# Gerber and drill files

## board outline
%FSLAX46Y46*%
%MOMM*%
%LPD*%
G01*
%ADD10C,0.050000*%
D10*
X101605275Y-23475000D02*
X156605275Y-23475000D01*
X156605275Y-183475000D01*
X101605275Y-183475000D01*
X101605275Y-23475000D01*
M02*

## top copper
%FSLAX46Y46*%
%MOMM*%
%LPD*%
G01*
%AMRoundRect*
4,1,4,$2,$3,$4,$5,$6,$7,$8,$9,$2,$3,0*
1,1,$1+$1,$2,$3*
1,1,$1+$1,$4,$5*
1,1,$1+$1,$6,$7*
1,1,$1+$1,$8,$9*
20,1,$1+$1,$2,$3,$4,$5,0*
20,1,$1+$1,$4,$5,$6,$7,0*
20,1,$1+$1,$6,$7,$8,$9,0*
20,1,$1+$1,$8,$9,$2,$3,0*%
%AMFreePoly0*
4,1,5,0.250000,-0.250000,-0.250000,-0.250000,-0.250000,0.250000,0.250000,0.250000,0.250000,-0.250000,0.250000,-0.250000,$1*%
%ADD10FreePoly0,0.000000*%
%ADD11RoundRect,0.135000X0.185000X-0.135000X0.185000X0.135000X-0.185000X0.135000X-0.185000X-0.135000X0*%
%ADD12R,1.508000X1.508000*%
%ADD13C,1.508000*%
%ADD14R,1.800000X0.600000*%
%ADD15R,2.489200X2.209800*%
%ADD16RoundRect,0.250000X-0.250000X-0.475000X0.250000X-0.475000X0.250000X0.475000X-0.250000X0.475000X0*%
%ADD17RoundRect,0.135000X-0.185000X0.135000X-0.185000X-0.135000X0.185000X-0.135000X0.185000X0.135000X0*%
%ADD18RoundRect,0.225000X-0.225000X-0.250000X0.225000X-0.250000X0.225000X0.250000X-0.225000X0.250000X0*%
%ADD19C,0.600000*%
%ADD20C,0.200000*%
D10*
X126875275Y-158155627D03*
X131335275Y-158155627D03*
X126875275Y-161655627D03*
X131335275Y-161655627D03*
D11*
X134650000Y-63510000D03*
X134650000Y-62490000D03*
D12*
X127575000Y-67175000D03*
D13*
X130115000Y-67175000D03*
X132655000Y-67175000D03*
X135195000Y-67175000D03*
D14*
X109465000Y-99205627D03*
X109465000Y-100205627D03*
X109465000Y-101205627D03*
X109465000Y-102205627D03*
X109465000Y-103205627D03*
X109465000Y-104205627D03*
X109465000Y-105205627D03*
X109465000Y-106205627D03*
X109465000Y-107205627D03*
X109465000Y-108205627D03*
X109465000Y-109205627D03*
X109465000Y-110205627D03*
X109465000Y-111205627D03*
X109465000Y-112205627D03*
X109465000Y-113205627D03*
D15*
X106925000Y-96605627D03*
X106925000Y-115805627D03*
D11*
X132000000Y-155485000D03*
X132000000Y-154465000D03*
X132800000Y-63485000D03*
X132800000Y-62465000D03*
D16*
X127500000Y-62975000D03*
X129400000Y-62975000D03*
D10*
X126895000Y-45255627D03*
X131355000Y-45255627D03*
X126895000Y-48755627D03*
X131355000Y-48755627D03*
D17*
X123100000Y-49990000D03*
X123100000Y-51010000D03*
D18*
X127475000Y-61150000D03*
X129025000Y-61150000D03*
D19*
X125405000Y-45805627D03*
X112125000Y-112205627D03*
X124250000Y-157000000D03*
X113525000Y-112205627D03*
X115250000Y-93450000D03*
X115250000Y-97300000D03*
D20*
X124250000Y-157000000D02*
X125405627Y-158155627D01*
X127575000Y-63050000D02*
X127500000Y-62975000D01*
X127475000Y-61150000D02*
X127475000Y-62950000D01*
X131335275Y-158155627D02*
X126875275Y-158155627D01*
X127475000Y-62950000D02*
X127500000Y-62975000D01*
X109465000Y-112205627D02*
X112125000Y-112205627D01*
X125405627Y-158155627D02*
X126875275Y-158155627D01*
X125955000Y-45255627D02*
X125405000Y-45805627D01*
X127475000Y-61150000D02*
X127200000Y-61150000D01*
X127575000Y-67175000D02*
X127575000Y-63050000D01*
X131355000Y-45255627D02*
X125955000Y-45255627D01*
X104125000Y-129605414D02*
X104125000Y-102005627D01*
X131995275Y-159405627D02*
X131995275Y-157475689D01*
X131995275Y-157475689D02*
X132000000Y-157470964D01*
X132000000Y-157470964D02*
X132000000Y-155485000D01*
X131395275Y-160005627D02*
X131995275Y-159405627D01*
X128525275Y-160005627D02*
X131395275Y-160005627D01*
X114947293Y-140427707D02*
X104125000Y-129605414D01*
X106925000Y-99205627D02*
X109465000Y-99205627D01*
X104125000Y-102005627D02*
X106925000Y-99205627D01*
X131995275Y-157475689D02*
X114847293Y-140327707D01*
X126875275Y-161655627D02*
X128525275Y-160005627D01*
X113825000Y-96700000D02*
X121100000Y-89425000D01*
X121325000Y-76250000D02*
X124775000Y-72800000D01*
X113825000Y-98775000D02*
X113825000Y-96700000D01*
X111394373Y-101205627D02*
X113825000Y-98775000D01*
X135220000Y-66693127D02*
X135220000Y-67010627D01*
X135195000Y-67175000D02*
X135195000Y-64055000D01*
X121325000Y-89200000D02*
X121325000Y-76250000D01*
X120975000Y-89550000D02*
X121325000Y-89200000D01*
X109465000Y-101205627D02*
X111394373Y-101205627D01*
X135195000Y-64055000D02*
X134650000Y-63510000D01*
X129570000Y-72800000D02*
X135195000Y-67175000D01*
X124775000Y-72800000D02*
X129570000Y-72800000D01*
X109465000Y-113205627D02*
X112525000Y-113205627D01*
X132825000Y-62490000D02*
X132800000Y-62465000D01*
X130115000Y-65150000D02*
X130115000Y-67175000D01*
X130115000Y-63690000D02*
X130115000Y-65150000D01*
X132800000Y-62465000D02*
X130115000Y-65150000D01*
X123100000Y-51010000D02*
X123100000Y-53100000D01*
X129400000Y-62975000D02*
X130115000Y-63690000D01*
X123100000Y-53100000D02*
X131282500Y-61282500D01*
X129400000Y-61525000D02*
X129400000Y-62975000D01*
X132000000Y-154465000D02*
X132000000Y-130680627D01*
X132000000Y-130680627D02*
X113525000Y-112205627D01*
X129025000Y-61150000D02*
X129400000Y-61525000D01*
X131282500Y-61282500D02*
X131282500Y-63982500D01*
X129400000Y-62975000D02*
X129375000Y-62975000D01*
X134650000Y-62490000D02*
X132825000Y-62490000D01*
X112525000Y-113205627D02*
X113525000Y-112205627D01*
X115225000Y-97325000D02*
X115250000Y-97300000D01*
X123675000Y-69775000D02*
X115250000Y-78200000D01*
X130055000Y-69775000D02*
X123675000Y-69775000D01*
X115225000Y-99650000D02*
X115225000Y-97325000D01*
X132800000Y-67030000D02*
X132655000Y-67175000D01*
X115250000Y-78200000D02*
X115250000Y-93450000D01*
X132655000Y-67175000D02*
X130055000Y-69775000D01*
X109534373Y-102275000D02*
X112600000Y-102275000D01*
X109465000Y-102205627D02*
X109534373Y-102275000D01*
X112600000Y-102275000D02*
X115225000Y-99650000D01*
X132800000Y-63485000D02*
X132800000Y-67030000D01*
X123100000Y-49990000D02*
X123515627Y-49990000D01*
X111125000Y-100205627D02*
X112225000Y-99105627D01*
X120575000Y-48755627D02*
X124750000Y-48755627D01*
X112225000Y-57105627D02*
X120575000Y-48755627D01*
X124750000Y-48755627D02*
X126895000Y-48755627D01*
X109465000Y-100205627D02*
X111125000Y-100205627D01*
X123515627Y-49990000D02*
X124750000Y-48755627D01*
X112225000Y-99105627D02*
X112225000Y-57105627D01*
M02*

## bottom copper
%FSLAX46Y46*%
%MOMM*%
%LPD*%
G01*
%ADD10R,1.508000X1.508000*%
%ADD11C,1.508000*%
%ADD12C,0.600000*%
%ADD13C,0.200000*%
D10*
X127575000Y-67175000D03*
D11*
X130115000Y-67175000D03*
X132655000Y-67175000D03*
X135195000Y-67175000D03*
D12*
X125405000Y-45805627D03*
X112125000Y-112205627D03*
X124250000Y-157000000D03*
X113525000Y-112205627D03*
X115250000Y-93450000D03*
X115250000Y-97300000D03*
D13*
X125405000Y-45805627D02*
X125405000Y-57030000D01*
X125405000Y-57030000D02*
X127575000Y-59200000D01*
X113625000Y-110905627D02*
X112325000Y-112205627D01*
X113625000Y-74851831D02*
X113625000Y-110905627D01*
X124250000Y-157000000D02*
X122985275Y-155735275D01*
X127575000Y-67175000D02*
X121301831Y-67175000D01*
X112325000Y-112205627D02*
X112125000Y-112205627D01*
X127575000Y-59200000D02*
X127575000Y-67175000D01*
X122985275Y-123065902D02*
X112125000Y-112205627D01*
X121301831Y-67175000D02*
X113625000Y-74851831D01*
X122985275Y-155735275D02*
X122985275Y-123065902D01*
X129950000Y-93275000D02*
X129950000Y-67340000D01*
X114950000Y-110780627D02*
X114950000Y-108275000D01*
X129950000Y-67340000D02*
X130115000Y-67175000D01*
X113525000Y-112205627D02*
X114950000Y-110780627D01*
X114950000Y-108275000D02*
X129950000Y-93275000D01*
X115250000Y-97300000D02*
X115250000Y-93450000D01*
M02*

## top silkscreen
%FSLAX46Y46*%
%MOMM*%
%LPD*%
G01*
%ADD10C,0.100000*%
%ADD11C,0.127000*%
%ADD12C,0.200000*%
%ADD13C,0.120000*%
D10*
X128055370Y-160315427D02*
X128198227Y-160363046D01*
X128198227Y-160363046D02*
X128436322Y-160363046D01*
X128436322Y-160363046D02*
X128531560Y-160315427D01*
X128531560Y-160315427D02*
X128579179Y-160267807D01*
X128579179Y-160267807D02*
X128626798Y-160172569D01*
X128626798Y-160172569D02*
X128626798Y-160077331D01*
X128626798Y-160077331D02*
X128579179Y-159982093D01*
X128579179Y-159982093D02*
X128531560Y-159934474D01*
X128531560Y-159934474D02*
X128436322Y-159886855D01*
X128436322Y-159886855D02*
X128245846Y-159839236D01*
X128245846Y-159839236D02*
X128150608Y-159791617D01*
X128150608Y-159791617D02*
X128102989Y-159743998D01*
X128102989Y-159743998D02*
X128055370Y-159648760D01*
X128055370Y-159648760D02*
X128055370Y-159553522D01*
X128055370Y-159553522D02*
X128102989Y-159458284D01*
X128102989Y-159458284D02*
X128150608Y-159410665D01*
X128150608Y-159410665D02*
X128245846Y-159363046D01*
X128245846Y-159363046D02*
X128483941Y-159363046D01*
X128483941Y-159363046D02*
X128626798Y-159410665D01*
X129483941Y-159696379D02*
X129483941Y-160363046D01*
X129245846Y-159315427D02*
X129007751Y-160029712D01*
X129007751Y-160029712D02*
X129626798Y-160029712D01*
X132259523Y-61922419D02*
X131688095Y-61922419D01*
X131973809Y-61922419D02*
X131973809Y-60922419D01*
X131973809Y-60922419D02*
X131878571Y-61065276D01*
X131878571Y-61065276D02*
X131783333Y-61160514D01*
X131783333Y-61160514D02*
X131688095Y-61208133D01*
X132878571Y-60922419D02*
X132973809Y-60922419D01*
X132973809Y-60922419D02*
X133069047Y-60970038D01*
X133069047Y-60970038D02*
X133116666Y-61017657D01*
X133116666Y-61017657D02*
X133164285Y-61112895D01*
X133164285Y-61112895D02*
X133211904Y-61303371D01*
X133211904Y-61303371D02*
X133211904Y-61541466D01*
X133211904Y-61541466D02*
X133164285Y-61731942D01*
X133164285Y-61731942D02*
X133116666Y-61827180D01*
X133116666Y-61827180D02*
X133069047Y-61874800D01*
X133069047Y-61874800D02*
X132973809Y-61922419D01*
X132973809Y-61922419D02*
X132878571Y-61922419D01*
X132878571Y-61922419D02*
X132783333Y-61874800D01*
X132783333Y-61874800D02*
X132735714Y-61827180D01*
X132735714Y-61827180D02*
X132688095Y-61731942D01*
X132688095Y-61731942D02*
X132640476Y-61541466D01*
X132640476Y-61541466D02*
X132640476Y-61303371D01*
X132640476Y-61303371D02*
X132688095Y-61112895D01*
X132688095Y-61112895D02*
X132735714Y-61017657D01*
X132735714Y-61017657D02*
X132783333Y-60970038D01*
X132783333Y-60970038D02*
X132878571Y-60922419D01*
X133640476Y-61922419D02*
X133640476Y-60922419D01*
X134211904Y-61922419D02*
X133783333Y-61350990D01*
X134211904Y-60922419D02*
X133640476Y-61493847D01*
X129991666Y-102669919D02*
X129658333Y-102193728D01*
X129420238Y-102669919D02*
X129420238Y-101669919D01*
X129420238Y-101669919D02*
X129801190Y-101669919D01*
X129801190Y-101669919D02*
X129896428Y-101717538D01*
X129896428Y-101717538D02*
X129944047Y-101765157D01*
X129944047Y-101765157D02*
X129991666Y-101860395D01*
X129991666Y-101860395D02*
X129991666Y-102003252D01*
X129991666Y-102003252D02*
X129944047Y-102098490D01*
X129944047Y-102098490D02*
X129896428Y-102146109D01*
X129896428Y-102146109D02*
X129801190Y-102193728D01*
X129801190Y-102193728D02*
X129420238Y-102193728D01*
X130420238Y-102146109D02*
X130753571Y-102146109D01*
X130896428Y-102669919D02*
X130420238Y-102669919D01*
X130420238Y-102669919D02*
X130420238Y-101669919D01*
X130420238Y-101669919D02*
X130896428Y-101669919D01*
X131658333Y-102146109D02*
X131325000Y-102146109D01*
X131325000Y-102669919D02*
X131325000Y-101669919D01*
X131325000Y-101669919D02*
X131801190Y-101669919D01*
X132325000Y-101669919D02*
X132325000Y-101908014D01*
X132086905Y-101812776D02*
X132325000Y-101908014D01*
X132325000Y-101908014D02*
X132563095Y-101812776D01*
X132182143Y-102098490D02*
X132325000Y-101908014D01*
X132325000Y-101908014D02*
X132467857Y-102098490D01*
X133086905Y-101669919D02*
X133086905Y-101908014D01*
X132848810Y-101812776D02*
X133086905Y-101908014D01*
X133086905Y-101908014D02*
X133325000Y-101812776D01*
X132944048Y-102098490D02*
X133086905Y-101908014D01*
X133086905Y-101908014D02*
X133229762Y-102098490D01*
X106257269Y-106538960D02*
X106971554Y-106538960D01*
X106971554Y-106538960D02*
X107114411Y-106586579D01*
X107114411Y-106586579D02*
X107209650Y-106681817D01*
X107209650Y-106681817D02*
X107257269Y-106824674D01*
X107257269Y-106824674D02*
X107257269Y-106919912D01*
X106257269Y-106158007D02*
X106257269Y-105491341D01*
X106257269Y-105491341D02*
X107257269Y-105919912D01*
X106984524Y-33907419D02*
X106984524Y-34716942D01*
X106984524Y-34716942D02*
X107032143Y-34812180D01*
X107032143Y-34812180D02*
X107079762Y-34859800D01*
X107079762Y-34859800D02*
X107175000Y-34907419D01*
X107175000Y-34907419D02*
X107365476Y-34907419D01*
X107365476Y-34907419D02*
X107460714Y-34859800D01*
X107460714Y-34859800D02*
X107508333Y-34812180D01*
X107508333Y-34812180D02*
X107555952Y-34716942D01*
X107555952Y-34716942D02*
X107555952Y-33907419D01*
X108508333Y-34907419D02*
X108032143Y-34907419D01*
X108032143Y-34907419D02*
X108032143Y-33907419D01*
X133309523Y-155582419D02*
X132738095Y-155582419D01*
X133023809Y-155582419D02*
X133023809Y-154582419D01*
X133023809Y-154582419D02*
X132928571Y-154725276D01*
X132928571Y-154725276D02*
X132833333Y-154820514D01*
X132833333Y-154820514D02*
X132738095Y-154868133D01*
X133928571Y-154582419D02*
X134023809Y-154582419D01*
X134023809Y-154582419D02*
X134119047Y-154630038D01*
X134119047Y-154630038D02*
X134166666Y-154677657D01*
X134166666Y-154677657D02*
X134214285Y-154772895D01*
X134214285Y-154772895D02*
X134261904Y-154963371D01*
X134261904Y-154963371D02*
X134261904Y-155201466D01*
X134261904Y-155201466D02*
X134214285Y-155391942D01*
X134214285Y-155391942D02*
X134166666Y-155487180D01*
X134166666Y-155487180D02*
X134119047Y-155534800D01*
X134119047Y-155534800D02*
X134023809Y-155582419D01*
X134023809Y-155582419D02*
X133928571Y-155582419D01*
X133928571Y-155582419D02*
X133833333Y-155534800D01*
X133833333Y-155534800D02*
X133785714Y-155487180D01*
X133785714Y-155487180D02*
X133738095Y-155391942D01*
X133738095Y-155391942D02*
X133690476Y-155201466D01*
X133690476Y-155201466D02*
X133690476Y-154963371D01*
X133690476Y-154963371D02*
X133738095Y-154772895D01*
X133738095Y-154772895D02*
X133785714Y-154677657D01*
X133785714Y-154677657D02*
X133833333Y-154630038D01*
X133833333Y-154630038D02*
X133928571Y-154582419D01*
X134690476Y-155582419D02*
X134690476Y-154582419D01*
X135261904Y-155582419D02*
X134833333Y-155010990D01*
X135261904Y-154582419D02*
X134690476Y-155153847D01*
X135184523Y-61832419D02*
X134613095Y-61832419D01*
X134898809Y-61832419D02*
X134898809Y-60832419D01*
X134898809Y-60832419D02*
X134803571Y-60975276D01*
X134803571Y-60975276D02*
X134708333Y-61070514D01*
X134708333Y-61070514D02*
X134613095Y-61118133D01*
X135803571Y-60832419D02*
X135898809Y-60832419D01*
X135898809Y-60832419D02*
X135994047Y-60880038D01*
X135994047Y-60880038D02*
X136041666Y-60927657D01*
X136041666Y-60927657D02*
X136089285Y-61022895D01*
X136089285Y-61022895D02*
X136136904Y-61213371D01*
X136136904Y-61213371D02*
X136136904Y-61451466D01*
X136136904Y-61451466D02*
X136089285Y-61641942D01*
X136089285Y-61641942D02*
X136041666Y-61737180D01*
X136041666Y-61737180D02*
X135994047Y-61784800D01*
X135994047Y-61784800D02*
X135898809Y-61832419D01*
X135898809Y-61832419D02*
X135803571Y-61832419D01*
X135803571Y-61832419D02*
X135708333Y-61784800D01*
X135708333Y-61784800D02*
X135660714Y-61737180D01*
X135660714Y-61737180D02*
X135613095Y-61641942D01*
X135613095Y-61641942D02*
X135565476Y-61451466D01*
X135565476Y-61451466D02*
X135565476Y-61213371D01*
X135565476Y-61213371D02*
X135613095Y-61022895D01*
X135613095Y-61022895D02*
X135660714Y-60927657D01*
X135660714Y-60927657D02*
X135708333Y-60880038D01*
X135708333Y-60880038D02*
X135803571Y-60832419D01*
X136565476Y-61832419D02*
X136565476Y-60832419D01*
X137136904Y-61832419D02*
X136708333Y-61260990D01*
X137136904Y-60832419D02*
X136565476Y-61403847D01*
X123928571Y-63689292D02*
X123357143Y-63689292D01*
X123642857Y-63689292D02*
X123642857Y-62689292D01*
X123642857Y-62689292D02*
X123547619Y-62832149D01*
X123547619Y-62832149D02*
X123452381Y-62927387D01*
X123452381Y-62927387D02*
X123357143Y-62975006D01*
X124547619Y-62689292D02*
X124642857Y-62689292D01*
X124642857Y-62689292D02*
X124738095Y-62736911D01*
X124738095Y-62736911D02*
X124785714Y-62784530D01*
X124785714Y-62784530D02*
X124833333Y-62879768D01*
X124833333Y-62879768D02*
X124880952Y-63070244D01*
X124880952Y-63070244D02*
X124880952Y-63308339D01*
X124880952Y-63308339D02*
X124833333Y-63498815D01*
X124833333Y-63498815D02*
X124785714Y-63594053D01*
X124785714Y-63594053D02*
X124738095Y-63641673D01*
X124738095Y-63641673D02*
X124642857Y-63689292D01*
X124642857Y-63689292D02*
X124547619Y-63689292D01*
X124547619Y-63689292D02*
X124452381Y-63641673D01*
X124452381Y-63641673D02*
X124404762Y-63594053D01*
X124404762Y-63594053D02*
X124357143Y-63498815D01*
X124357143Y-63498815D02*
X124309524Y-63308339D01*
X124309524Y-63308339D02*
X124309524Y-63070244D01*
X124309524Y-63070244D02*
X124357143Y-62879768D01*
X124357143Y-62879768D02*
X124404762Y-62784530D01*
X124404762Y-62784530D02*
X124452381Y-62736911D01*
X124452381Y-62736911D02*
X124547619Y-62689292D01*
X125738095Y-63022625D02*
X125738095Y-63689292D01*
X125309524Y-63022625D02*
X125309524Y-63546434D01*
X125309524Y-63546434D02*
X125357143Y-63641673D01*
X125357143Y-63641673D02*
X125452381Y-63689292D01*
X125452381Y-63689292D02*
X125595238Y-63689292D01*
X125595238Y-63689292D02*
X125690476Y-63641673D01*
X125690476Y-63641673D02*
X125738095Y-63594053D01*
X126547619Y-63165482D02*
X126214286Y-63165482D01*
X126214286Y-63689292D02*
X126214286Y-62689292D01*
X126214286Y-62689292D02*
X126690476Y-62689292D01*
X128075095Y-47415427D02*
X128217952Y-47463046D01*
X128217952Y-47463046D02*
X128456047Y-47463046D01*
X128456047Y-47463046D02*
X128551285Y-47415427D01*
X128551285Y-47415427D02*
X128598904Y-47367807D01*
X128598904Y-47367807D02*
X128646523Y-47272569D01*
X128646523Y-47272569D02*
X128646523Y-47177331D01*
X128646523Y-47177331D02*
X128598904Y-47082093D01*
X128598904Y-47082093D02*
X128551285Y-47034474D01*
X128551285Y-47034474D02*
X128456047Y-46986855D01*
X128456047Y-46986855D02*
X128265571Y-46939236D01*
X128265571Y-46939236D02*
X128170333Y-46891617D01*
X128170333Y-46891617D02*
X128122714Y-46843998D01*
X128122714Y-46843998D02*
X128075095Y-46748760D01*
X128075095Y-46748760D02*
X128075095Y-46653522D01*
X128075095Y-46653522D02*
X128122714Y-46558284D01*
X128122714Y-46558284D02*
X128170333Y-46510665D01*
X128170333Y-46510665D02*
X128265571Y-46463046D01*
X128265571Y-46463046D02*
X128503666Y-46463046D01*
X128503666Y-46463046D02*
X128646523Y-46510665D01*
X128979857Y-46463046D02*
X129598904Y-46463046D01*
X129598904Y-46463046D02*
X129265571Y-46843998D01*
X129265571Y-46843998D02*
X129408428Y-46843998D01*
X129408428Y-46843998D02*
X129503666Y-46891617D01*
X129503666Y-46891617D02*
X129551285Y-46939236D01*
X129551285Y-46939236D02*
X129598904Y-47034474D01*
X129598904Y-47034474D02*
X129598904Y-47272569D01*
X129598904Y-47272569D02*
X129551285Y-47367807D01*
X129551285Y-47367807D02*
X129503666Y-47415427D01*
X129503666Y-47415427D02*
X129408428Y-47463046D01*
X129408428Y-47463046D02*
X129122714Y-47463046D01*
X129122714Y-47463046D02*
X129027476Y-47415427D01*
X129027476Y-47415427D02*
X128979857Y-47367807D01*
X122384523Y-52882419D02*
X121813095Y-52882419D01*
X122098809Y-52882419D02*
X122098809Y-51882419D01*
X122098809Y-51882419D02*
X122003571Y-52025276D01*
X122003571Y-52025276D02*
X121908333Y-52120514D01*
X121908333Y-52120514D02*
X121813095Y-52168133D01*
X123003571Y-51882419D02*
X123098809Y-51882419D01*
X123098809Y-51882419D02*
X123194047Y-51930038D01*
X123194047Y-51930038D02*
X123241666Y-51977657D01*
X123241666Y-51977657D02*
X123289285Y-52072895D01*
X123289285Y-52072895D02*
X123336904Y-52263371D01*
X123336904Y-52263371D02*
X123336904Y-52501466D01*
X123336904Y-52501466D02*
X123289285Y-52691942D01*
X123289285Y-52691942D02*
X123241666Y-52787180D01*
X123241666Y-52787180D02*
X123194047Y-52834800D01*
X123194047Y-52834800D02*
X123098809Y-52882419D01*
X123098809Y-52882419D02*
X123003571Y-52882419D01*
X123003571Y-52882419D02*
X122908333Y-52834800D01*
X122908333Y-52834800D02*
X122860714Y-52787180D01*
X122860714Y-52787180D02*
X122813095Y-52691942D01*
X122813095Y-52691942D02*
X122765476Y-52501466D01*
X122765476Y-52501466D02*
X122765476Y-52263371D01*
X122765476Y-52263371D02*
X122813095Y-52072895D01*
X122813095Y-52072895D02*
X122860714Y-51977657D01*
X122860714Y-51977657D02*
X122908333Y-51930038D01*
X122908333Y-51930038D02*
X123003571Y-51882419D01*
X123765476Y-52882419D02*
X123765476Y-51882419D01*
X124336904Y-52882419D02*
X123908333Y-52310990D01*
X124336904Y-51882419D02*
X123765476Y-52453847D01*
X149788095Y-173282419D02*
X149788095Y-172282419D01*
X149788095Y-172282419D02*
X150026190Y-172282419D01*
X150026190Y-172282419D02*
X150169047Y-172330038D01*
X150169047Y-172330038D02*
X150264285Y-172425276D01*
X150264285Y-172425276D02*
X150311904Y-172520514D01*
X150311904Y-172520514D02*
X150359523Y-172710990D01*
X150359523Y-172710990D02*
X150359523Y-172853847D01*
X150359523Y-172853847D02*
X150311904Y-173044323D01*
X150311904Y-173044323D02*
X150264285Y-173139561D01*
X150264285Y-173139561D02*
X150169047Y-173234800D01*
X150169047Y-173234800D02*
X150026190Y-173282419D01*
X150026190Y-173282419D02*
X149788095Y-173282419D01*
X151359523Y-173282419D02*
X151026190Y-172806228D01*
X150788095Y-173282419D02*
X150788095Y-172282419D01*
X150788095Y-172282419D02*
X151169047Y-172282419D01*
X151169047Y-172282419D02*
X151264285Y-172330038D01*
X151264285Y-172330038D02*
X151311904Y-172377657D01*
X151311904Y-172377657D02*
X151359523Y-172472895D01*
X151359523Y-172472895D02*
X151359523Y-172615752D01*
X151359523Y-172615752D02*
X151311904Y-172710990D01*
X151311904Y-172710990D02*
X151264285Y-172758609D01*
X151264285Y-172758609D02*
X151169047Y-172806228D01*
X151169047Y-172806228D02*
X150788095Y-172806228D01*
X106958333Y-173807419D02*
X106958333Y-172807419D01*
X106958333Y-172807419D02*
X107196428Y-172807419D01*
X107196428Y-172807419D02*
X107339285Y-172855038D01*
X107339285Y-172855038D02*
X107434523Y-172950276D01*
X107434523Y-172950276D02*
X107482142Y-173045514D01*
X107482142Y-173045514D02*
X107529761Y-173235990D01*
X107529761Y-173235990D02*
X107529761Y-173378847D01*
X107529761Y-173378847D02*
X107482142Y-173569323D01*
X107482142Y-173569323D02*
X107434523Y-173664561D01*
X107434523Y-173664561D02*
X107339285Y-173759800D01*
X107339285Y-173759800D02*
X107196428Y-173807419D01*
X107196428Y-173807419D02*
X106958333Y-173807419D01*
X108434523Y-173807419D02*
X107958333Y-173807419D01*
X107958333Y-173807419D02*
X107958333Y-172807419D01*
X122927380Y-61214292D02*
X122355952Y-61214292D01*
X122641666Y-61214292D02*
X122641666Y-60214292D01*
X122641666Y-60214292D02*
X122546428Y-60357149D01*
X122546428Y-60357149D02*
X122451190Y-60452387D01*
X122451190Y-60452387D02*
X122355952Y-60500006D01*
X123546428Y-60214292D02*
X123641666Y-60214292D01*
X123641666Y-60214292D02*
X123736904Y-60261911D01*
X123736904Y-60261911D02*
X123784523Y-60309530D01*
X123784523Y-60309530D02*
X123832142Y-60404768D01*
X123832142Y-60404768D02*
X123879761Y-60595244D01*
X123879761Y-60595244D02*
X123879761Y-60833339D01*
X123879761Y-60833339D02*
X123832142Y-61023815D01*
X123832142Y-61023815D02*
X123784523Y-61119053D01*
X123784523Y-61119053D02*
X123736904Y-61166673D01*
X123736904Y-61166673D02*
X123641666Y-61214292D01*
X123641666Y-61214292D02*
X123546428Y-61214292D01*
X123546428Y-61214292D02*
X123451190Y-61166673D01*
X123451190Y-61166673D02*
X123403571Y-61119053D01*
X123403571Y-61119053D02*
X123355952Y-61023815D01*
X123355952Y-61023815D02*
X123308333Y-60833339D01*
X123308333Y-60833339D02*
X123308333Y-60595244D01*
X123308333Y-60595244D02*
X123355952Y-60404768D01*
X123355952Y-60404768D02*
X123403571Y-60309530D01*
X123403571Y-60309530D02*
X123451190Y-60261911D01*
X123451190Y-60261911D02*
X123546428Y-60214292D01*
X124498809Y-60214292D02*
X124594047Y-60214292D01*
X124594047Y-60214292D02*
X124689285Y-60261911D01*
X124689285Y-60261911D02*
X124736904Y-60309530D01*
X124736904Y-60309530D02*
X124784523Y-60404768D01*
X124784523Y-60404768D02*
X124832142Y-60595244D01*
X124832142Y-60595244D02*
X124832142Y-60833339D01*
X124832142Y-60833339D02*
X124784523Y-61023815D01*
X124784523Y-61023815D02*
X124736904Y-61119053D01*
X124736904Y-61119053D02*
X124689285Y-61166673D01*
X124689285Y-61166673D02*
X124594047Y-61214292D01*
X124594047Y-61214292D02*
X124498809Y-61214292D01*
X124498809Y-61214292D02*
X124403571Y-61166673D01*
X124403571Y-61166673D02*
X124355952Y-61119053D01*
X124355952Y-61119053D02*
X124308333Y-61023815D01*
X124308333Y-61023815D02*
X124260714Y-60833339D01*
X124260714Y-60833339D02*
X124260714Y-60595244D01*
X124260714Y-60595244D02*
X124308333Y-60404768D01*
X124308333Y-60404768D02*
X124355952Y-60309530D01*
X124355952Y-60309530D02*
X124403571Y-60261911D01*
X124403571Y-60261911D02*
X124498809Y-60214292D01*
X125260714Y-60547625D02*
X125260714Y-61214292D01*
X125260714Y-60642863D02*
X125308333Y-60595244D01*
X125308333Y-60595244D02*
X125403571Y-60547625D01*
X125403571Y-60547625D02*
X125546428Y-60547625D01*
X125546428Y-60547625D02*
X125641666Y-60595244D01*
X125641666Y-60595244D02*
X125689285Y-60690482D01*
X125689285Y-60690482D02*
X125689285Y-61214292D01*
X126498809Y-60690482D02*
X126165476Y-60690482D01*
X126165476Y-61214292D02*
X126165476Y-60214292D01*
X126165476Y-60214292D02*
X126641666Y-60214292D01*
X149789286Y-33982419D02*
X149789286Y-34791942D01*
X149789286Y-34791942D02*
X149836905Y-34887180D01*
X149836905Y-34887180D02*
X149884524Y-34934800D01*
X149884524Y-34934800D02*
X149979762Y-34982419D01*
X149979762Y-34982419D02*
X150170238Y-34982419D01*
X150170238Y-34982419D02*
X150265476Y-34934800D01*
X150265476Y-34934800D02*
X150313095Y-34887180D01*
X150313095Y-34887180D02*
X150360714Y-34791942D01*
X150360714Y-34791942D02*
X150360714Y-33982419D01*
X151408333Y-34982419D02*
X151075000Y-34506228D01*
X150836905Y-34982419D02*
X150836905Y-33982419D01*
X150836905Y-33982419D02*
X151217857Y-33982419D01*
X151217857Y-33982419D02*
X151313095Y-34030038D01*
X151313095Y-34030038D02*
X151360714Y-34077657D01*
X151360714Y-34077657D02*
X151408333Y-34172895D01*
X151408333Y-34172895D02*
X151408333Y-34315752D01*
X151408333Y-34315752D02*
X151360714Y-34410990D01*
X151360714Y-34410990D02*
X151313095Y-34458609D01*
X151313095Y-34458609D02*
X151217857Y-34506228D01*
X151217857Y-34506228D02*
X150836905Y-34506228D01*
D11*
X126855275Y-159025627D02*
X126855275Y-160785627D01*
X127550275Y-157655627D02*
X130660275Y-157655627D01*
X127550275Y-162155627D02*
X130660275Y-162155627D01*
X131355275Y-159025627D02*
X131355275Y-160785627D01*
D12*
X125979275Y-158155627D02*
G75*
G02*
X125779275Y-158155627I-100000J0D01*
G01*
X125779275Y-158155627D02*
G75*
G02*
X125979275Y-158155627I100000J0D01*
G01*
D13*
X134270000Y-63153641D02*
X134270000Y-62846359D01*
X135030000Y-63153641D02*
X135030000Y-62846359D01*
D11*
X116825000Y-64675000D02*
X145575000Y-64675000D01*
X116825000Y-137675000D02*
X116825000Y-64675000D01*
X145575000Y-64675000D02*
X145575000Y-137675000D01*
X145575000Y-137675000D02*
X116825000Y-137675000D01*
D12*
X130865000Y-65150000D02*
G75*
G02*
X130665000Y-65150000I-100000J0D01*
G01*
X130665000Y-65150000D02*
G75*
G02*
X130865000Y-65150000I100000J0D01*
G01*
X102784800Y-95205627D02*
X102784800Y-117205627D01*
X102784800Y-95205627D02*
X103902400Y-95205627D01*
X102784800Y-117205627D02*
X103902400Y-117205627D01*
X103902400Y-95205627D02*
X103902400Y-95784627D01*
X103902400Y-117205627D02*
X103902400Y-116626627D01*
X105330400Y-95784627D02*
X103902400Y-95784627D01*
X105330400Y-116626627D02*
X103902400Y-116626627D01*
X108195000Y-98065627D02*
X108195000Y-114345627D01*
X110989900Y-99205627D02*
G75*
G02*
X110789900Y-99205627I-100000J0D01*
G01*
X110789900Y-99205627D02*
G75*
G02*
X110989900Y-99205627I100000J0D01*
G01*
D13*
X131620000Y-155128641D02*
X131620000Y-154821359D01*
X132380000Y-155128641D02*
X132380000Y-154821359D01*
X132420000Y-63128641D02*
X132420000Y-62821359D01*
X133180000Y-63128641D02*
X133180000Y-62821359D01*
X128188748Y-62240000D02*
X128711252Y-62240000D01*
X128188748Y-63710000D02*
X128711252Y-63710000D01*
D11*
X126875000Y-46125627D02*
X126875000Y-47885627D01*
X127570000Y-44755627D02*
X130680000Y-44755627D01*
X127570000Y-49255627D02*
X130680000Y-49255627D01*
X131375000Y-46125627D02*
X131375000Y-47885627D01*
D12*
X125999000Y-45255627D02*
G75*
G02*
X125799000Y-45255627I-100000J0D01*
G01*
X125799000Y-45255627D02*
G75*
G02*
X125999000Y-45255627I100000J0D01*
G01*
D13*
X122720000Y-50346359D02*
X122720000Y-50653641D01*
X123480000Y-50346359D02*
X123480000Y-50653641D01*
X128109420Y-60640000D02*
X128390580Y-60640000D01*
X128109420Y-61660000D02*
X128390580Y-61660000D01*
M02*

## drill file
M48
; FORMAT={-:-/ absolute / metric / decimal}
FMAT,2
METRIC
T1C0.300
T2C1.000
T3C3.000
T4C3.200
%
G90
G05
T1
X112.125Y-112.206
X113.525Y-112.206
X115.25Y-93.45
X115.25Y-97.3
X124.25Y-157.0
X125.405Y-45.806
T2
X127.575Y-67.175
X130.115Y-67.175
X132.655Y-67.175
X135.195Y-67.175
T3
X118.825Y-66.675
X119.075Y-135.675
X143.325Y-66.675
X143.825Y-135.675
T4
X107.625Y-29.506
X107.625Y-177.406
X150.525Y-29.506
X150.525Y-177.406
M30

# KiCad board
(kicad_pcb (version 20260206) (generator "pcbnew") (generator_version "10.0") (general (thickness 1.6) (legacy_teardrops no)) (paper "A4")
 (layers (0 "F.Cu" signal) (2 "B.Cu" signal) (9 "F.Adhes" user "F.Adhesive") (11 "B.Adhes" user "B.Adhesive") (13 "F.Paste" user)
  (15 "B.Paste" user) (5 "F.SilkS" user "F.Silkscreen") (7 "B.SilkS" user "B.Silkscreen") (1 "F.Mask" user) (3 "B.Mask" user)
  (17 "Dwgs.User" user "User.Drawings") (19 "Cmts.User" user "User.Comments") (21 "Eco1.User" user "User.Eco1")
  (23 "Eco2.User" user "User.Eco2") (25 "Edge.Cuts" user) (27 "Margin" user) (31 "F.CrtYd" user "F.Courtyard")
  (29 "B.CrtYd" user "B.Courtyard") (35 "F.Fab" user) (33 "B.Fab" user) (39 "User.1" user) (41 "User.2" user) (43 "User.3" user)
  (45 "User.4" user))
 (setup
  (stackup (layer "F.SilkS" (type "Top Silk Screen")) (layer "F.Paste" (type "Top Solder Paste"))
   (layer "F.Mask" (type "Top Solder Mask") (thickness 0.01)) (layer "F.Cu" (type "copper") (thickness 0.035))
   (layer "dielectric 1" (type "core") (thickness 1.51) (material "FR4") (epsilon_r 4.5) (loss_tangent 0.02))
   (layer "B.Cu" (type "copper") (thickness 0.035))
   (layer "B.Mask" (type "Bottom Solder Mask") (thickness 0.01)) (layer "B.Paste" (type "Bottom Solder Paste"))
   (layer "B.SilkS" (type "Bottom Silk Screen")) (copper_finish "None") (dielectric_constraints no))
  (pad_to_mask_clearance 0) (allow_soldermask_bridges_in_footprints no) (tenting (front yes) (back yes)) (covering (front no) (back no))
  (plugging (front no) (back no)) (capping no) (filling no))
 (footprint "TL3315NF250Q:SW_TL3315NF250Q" (layer "F.Cu") (at 129.105275 159.905627)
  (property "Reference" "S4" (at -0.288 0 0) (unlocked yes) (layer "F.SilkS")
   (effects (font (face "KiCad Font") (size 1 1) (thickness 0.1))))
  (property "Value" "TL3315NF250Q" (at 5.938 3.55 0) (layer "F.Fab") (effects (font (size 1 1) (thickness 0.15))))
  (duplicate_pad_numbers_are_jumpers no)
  (fp_line (start -2.25 -0.88) (end -2.25 0.88) (stroke (width 0.127) (type solid)) (layer "F.SilkS"))
  (fp_line (start -1.555 -2.25) (end 1.555 -2.25) (stroke (width 0.127) (type solid)) (layer "F.SilkS"))
  (fp_line (start -1.555 2.25) (end 1.555 2.25) (stroke (width 0.127) (type solid)) (layer "F.SilkS"))
  (fp_line (start 2.25 -0.88) (end 2.25 0.88) (stroke (width 0.127) (type solid)) (layer "F.SilkS"))
  (fp_circle (center -3.226 -1.75) (end -3.126 -1.75) (stroke (width 0.2) (type solid)) (fill no) (layer "F.SilkS"))
  (pad "1" smd custom (at -2.23 -1.75) (size 0.5 0.5) (layers "F.Cu") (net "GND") (options (clearance outline) (anchor rect)) (primitives))
  (pad "2" smd custom (at 2.23 -1.75) (size 0.5 0.5) (layers "F.Cu") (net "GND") (options (clearance outline) (anchor rect)) (primitives))
  (pad "3" smd custom (at -2.23 1.75) (size 0.5 0.5) (layers "F.Cu") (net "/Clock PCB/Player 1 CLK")
   (options (clearance outline) (anchor rect)) (primitives))
  (pad "4" smd custom (at 2.23 1.75) (size 0.5 0.5) (layers "F.Cu") (options (clearance outline) (anchor rect)) (primitives)))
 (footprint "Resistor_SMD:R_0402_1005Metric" (layer "F.Cu") (at 134.65 63 90)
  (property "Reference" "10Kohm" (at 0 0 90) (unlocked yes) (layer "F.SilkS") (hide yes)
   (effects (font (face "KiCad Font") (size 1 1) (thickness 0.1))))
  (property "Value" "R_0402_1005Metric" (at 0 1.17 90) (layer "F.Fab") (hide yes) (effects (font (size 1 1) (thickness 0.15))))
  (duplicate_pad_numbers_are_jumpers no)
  (fp_line (start -0.153641 -0.38) (end 0.153641 -0.38) (stroke (width 0.12) (type solid)) (layer "F.SilkS"))
  (fp_line (start -0.153641 0.38) (end 0.153641 0.38) (stroke (width 0.12) (type solid)) (layer "F.SilkS"))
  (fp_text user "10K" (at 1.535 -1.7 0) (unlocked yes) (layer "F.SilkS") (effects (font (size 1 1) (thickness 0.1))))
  (pad "1" smd roundrect (at -0.51 0 90) (size 0.54 0.64) (layers "F.Cu" "F.Mask" "F.Paste") (roundrect_rratio 0.25) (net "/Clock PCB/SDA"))
  (pad "2" smd roundrect (at 0.51 0 90) (size 0.54 0.64) (layers "F.Cu" "F.Mask" "F.Paste") (roundrect_rratio 0.25) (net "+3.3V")))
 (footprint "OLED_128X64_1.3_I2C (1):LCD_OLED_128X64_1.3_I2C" (layer "F.Cu") (at 131.325 101.675)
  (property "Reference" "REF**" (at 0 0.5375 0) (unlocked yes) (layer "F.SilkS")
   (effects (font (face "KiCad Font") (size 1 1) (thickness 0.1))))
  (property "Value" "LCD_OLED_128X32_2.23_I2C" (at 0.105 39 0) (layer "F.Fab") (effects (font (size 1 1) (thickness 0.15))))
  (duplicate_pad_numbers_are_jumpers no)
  (fp_line (start -14.5 -37) (end 14.25 -37) (stroke (width 0.127) (type solid)) (layer "F.SilkS"))
  (fp_line (start -14.5 36) (end -14.5 -37) (stroke (width 0.127) (type solid)) (layer "F.SilkS"))
  (fp_line (start 14.25 -37) (end 14.25 36) (stroke (width 0.127) (type solid)) (layer "F.SilkS"))
  (fp_line (start 14.25 36) (end -14.5 36) (stroke (width 0.127) (type solid)) (layer "F.SilkS"))
  (fp_circle (center -0.56 -36.525) (end -0.46 -36.525) (stroke (width 0.2) (type solid)) (fill no) (layer "F.SilkS"))
  (pad "" np_thru_hole circle (at -12.5 -35) (size 3 3) (drill 3) (layers "*.Cu" "*.Mask"))
  (pad "" np_thru_hole circle (at -12.25 34) (size 3 3) (drill 3) (layers "*.Cu" "*.Mask"))
  (pad "" np_thru_hole circle (at 12 -35) (size 3 3) (drill 3) (layers "*.Cu" "*.Mask"))
  (pad "" np_thru_hole circle (at 12.5 34) (size 3 3) (drill 3) (layers "*.Cu" "*.Mask"))
  (pad "1" thru_hole rect (at -3.75 -34.5) (size 1.508 1.508) (drill 1) (layers "*.Cu" "*.Mask") (remove_unused_layers no) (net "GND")
   (solder_mask_margin 0.102))
  (pad "2" thru_hole circle (at -1.21 -34.5) (size 1.508 1.508) (drill 1) (layers "*.Cu" "*.Mask") (remove_unused_layers no) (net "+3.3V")
   (solder_mask_margin 0.102))
  (pad "3" thru_hole circle (at 1.33 -34.5) (size 1.508 1.508) (drill 1) (layers "*.Cu" "*.Mask") (remove_unused_layers no) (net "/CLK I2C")
   (solder_mask_margin 0.102))
  (pad "4" thru_hole circle (at 3.87 -34.5) (size 1.508 1.508) (drill 1) (layers "*.Cu" "*.Mask") (remove_unused_layers no)
   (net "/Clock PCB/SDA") (solder_mask_margin 0.102)))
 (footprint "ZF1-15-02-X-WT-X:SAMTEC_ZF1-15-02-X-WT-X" (layer "F.Cu") (at 105.4899 106.205627 -90)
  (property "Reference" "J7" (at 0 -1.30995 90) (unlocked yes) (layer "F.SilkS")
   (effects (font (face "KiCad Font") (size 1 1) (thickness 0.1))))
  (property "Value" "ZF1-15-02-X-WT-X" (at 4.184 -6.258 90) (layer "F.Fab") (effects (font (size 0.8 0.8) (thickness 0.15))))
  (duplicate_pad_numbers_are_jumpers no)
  (fp_line (start -11 2.7051) (end 11 2.7051) (stroke (width 0.2) (type solid)) (layer "F.SilkS"))
  (fp_line (start -11 2.7051) (end -11 1.5875) (stroke (width 0.2) (type solid)) (layer "F.SilkS"))
  (fp_line (start 11 2.7051) (end 11 1.5875) (stroke (width 0.2) (type solid)) (layer "F.SilkS"))
  (fp_line (start -11 1.5875) (end -10.421 1.5875) (stroke (width 0.2) (type solid)) (layer "F.SilkS"))
  (fp_line (start 11 1.5875) (end 10.421 1.5875) (stroke (width 0.2) (type solid)) (layer "F.SilkS"))
  (fp_line (start -10.421 0.1595) (end -10.421 1.5875) (stroke (width 0.2) (type solid)) (layer "F.SilkS"))
  (fp_line (start 10.421 0.1595) (end 10.421 1.5875) (stroke (width 0.2) (type solid)) (layer "F.SilkS"))
  (fp_line (start -8.14 -2.7051) (end 8.14 -2.7051) (stroke (width 0.2) (type solid)) (layer "F.SilkS"))
  (fp_circle (center -7 -5.4) (end -6.9 -5.4) (stroke (width 0.2) (type solid)) (fill no) (layer "F.SilkS"))
  (pad "01" smd rect (at -7 -3.9751 270) (size 0.6 1.8) (layers "F.Cu" "F.Mask" "F.Paste") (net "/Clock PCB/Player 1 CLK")
   (solder_mask_margin 0.102))
  (pad "02" smd rect (at -6 -3.9751 270) (size 0.6 1.8) (layers "F.Cu" "F.Mask" "F.Paste") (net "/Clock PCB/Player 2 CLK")
   (solder_mask_margin 0.102))
  (pad "03" smd rect (at -5 -3.9751 270) (size 0.6 1.8) (layers "F.Cu" "F.Mask" "F.Paste") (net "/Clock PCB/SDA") (solder_mask_margin 0.102))
  (pad "04" smd rect (at -4 -3.9751 270) (size 0.6 1.8) (layers "F.Cu" "F.Mask" "F.Paste") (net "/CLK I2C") (solder_mask_margin 0.102))
  (pad "05" smd rect (at -3 -3.9751 270) (size 0.6 1.8) (layers "F.Cu" "F.Mask" "F.Paste") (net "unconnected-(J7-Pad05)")
   (solder_mask_margin 0.102))
  (pad "06" smd rect (at -2 -3.9751 270) (size 0.6 1.8) (layers "F.Cu" "F.Mask" "F.Paste") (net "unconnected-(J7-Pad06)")
   (solder_mask_margin 0.102))
  (pad "07" smd rect (at -1 -3.9751 270) (size 0.6 1.8) (layers "F.Cu" "F.Mask" "F.Paste") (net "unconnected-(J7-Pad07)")
   (solder_mask_margin 0.102))
  (pad "08" smd rect (at 0 -3.9751 270) (size 0.6 1.8) (layers "F.Cu" "F.Mask" "F.Paste") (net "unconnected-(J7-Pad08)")
   (solder_mask_margin 0.102))
  (pad "09" smd rect (at 1 -3.9751 270) (size 0.6 1.8) (layers "F.Cu" "F.Mask" "F.Paste") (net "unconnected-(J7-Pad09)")
   (solder_mask_margin 0.102))
  (pad "10" smd rect (at 2 -3.9751 270) (size 0.6 1.8) (layers "F.Cu" "F.Mask" "F.Paste") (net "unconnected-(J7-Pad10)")
   (solder_mask_margin 0.102))
  (pad "11" smd rect (at 3 -3.9751 270) (size 0.6 1.8) (layers "F.Cu" "F.Mask" "F.Paste") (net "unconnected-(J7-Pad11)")
   (solder_mask_margin 0.102))
  (pad "12" smd rect (at 4 -3.9751 270) (size 0.6 1.8) (layers "F.Cu" "F.Mask" "F.Paste") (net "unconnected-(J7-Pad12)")
   (solder_mask_margin 0.102))
  (pad "13" smd rect (at 5 -3.9751 270) (size 0.6 1.8) (layers "F.Cu" "F.Mask" "F.Paste") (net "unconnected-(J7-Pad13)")
   (solder_mask_margin 0.102))
  (pad "14" smd rect (at 6 -3.9751 270) (size 0.6 1.8) (layers "F.Cu" "F.Mask" "F.Paste") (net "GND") (solder_mask_margin 0.102))
  (pad "15" smd rect (at 7 -3.9751 270) (size 0.6 1.8) (layers "F.Cu" "F.Mask" "F.Paste") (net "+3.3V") (solder_mask_margin 0.102))
  (pad "MP1" smd rect (at -9.6 -1.4351 270) (size 2.2098 2.4892) (layers "F.Cu" "F.Mask" "F.Paste") (solder_mask_margin 0.102))
  (pad "MP2" smd rect (at 9.6 -1.4351 270) (size 2.2098 2.4892) (layers "F.Cu" "F.Mask" "F.Paste") (solder_mask_margin 0.102)))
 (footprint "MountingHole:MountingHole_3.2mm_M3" (layer "F.Cu") (at 107.625 29.505627)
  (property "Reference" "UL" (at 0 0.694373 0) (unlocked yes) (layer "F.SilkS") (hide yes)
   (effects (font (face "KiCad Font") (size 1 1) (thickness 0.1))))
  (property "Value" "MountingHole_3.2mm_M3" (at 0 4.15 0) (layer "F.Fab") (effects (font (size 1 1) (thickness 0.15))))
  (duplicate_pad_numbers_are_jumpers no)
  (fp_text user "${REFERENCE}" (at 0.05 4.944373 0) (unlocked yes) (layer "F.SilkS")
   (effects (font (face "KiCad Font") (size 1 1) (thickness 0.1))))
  (pad "" np_thru_hole circle (at 0 0) (size 3.2 3.2) (drill 3.2) (layers "*.Cu" "*.Mask")))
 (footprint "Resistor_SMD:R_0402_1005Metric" (layer "F.Cu") (at 132 154.975 90)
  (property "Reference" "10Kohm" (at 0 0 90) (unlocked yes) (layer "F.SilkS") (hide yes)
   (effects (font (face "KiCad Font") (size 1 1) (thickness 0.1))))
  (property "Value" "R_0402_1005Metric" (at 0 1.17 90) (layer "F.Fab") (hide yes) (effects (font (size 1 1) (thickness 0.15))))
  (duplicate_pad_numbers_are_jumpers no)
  (fp_line (start -0.153641 -0.38) (end 0.153641 -0.38) (stroke (width 0.12) (type solid)) (layer "F.SilkS"))
  (fp_line (start -0.153641 0.38) (end 0.153641 0.38) (stroke (width 0.12) (type solid)) (layer "F.SilkS"))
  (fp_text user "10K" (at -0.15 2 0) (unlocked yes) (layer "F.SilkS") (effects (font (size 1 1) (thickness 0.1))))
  (pad "1" smd roundrect (at -0.51 0 90) (size 0.54 0.64) (layers "F.Cu" "F.Mask" "F.Paste") (roundrect_rratio 0.25)
   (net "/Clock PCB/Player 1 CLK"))
  (pad "2" smd roundrect (at 0.51 0 90) (size 0.54 0.64) (layers "F.Cu" "F.Mask" "F.Paste") (roundrect_rratio 0.25) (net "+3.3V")))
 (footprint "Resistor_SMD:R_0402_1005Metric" (layer "F.Cu") (at 132.8 62.975 90)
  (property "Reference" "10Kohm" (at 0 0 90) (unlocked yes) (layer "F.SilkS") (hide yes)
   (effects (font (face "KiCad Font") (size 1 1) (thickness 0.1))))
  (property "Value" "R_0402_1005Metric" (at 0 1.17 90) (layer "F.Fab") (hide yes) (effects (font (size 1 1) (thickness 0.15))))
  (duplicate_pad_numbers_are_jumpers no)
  (fp_line (start -0.153641 -0.38) (end 0.153641 -0.38) (stroke (width 0.12) (type solid)) (layer "F.SilkS"))
  (fp_line (start -0.153641 0.38) (end 0.153641 0.38) (stroke (width 0.12) (type solid)) (layer "F.SilkS"))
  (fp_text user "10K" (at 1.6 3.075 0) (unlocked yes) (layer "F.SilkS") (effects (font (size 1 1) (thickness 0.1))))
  (pad "1" smd roundrect (at -0.51 0 90) (size 0.54 0.64) (layers "F.Cu" "F.Mask" "F.Paste") (roundrect_rratio 0.25) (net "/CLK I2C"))
  (pad "2" smd roundrect (at 0.51 0 90) (size 0.54 0.64) (layers "F.Cu" "F.Mask" "F.Paste") (roundrect_rratio 0.25) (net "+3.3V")))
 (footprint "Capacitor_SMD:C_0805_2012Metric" (layer "F.Cu") (at 128.45 62.975)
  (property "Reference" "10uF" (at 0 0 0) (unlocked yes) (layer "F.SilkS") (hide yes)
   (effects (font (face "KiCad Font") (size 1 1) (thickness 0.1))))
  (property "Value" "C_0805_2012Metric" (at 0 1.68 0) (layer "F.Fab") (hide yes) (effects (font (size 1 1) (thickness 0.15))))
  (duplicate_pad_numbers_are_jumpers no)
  (fp_line (start -0.261252 -0.735) (end 0.261252 -0.735) (stroke (width 0.12) (type solid)) (layer "F.SilkS"))
  (fp_line (start -0.261252 0.735) (end 0.261252 0.735) (stroke (width 0.12) (type solid)) (layer "F.SilkS"))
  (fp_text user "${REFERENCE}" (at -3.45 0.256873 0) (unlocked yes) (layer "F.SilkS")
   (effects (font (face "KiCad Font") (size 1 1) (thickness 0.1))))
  (pad "1" smd roundrect (at -0.95 0) (size 1 1.45) (layers "F.Cu" "F.Mask" "F.Paste") (roundrect_rratio 0.25) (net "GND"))
  (pad "2" smd roundrect (at 0.95 0) (size 1 1.45) (layers "F.Cu" "F.Mask" "F.Paste") (roundrect_rratio 0.25) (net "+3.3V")))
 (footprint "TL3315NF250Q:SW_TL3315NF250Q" (layer "F.Cu") (at 129.125 47.005627)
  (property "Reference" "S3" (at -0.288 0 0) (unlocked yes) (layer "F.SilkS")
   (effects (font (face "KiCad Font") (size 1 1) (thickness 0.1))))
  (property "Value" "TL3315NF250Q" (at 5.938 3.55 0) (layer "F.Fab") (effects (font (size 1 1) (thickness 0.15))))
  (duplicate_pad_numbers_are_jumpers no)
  (fp_line (start -2.25 -0.88) (end -2.25 0.88) (stroke (width 0.127) (type solid)) (layer "F.SilkS"))
  (fp_line (start -1.555 -2.25) (end 1.555 -2.25) (stroke (width 0.127) (type solid)) (layer "F.SilkS"))
  (fp_line (start -1.555 2.25) (end 1.555 2.25) (stroke (width 0.127) (type solid)) (layer "F.SilkS"))
  (fp_line (start 2.25 -0.88) (end 2.25 0.88) (stroke (width 0.127) (type solid)) (layer "F.SilkS"))
  (fp_circle (center -3.226 -1.75) (end -3.126 -1.75) (stroke (width 0.2) (type solid)) (fill no) (layer "F.SilkS"))
  (pad "1" smd custom (at -2.23 -1.75) (size 0.5 0.5) (layers "F.Cu") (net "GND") (options (clearance outline) (anchor rect)) (primitives))
  (pad "2" smd custom (at 2.23 -1.75) (size 0.5 0.5) (layers "F.Cu") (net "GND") (options (clearance outline) (anchor rect)) (primitives))
  (pad "3" smd custom (at -2.23 1.75) (size 0.5 0.5) (layers "F.Cu") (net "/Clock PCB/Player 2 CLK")
   (options (clearance outline) (anchor rect)) (primitives))
  (pad "4" smd custom (at 2.23 1.75) (size 0.5 0.5) (layers "F.Cu") (options (clearance outline) (anchor rect)) (primitives)))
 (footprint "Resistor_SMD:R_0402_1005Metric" (layer "F.Cu") (at 123.1 50.5 -90)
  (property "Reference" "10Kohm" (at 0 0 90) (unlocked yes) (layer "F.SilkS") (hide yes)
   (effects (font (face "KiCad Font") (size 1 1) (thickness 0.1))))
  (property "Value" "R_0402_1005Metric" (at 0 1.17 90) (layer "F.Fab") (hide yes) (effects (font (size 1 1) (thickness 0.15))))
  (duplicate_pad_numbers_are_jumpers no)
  (fp_line (start -0.153641 0.38) (end 0.153641 0.38) (stroke (width 0.12) (type solid)) (layer "F.SilkS"))
  (fp_line (start -0.153641 -0.38) (end 0.153641 -0.38) (stroke (width 0.12) (type solid)) (layer "F.SilkS"))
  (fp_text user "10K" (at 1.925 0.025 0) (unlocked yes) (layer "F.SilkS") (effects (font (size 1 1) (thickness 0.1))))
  (pad "1" smd roundrect (at -0.51 0 270) (size 0.54 0.64) (layers "F.Cu" "F.Mask" "F.Paste") (roundrect_rratio 0.25)
   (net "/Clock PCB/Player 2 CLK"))
  (pad "2" smd roundrect (at 0.51 0 270) (size 0.54 0.64) (layers "F.Cu" "F.Mask" "F.Paste") (roundrect_rratio 0.25) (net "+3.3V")))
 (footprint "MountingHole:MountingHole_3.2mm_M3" (layer "F.Cu") (at 150.525 177.405627)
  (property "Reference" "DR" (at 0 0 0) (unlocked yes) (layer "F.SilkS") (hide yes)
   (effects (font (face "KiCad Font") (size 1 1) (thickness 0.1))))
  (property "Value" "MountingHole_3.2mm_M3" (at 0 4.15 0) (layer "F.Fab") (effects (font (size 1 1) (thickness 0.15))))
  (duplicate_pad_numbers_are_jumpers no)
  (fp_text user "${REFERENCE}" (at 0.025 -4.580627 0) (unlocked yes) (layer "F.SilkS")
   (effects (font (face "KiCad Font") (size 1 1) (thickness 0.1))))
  (pad "" np_thru_hole circle (at 0 0) (size 3.2 3.2) (drill 3.2) (layers "*.Cu" "*.Mask")))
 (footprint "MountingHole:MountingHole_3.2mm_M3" (layer "F.Cu") (at 107.625 177.405627)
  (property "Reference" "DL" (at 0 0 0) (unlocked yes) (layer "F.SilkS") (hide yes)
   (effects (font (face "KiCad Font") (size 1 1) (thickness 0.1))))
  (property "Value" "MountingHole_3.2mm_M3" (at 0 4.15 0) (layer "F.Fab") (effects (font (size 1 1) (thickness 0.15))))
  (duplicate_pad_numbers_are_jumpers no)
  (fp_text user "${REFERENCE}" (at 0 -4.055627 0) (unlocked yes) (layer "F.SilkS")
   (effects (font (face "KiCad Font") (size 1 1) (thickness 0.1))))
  (pad "" np_thru_hole circle (at 0 0) (size 3.2 3.2) (drill 3.2) (layers "*.Cu" "*.Mask")))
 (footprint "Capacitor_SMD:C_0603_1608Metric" (layer "F.Cu") (at 128.25 61.15)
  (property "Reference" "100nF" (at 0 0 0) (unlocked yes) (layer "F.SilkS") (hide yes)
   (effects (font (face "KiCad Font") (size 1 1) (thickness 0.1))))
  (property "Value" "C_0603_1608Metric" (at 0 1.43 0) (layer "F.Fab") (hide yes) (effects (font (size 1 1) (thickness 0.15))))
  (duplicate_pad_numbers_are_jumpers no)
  (fp_line (start -0.14058 -0.51) (end 0.14058 -0.51) (stroke (width 0.12) (type solid)) (layer "F.SilkS"))
  (fp_line (start -0.14058 0.51) (end 0.14058 0.51) (stroke (width 0.12) (type solid)) (layer "F.SilkS"))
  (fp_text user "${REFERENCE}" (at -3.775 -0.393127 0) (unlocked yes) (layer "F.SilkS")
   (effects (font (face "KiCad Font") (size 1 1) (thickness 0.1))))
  (pad "1" smd roundrect (at -0.775 0) (size 0.9 0.95) (layers "F.Cu" "F.Mask" "F.Paste") (roundrect_rratio 0.25) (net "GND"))
  (pad "2" smd roundrect (at 0.775 0) (size 0.9 0.95) (layers "F.Cu" "F.Mask" "F.Paste") (roundrect_rratio 0.25) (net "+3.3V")))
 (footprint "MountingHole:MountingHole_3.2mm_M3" (layer "F.Cu") (at 150.525 29.505627)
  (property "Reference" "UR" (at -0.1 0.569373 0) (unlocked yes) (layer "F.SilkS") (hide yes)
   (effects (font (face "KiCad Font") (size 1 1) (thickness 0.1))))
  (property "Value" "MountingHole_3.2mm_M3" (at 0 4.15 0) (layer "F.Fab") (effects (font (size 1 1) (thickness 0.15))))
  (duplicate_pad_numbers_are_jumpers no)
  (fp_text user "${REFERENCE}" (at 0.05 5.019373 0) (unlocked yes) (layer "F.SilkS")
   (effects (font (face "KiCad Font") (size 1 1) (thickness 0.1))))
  (pad "" np_thru_hole circle (at 0 0) (size 3.2 3.2) (drill 3.2) (layers "*.Cu" "*.Mask")))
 (gr_rect (start 101.605275 23.475) (end 156.605275 183.475) (stroke (width 0.05) (type solid)) (fill no) (layer "Edge.Cuts"))
 (segment (start 124.25 157) (end 125.405627 158.155627) (width 0.2) (layer "F.Cu") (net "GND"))
 (segment (start 127.575 63.05) (end 127.5 62.975) (width 0.2) (layer "F.Cu") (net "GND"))
 (segment (start 127.475 61.15) (end 127.475 62.95) (width 0.2) (layer "F.Cu") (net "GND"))
 (segment (start 131.335275 158.155627) (end 126.875275 158.155627) (width 0.2) (layer "F.Cu") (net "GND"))
 (segment (start 127.475 62.95) (end 127.5 62.975) (width 0.2) (layer "F.Cu") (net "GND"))
 (segment (start 109.465 112.205627) (end 112.125 112.205627) (width 0.2) (layer "F.Cu") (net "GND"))
 (segment (start 125.405627 158.155627) (end 126.875275 158.155627) (width 0.2) (layer "F.Cu") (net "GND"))
 (segment (start 125.955 45.255627) (end 125.405 45.805627) (width 0.2) (layer "F.Cu") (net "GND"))
 (segment (start 127.475 61.15) (end 127.2 61.15) (width 0.2) (layer "F.Cu") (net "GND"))
 (segment (start 127.575 67.175) (end 127.575 63.05) (width 0.2) (layer "F.Cu") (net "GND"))
 (segment (start 131.355 45.255627) (end 125.955 45.255627) (width 0.2) (layer "F.Cu") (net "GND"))
 (via (at 125.405 45.805627) (size 0.6) (drill 0.3) (layers "F.Cu" "B.Cu") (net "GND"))
 (via (at 112.125 112.205627) (size 0.6) (drill 0.3) (layers "F.Cu" "B.Cu") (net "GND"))
 (via (at 124.25 157) (size 0.6) (drill 0.3) (layers "F.Cu" "B.Cu") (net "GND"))
 (segment (start 125.405 45.805627) (end 125.405 57.03) (width 0.2) (layer "B.Cu") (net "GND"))
 (segment (start 125.405 57.03) (end 127.575 59.2) (width 0.2) (layer "B.Cu") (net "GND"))
 (segment (start 113.625 110.905627) (end 112.325 112.205627) (width 0.2) (layer "B.Cu") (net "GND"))
 (segment (start 113.625 74.851831) (end 113.625 110.905627) (width 0.2) (layer "B.Cu") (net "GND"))
 (segment (start 124.25 157) (end 122.985275 155.735275) (width 0.2) (layer "B.Cu") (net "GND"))
 (segment (start 127.575 67.175) (end 121.301831 67.175) (width 0.2) (layer "B.Cu") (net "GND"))
 (segment (start 112.325 112.205627) (end 112.125 112.205627) (width 0.2) (layer "B.Cu") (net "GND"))
 (segment (start 127.575 59.2) (end 127.575 67.175) (width 0.2) (layer "B.Cu") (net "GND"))
 (segment (start 122.985275 123.065902) (end 112.125 112.205627) (width 0.2) (layer "B.Cu") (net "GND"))
 (segment (start 121.301831 67.175) (end 113.625 74.851831) (width 0.2) (layer "B.Cu") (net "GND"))
 (segment (start 122.985275 155.735275) (end 122.985275 123.065902) (width 0.2) (layer "B.Cu") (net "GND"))
 (segment (start 104.125 129.605414) (end 104.125 102.005627) (width 0.2) (layer "F.Cu") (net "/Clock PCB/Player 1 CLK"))
 (segment (start 131.995275 159.405627) (end 131.995275 157.475689) (width 0.2) (layer "F.Cu") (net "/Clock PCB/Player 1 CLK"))
 (segment (start 131.995275 157.475689) (end 132 157.470964) (width 0.2) (layer "F.Cu") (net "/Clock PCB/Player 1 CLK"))
 (segment (start 132 157.470964) (end 132 155.485) (width 0.2) (layer "F.Cu") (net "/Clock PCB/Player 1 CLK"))
 (segment (start 131.395275 160.005627) (end 131.995275 159.405627) (width 0.2) (layer "F.Cu") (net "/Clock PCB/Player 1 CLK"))
 (segment (start 128.525275 160.005627) (end 131.395275 160.005627) (width 0.2) (layer "F.Cu") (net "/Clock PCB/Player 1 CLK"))
 (segment (start 114.947293 140.427707) (end 104.125 129.605414) (width 0.2) (layer "F.Cu") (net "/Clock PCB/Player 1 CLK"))
 (segment (start 106.925 99.205627) (end 109.465 99.205627) (width 0.2) (layer "F.Cu") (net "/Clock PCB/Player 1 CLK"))
 (segment (start 104.125 102.005627) (end 106.925 99.205627) (width 0.2) (layer "F.Cu") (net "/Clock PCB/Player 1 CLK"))
 (segment (start 131.995275 157.475689) (end 114.847293 140.327707) (width 0.2) (layer "F.Cu") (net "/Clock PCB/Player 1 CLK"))
 (segment (start 126.875275 161.655627) (end 128.525275 160.005627) (width 0.2) (layer "F.Cu") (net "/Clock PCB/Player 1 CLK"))
 (segment (start 113.825 96.7) (end 121.1 89.425) (width 0.2) (layer "F.Cu") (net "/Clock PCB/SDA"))
 (segment (start 121.325 76.25) (end 124.775 72.8) (width 0.2) (layer "F.Cu") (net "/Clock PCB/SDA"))
 (segment (start 113.825 98.775) (end 113.825 96.7) (width 0.2) (layer "F.Cu") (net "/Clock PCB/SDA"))
 (segment (start 111.394373 101.205627) (end 113.825 98.775) (width 0.2) (layer "F.Cu") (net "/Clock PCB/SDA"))
 (segment (start 135.22 66.693127) (end 135.22 67.010627) (width 0.2) (layer "F.Cu") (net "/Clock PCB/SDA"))
 (segment (start 135.195 67.175) (end 135.195 64.055) (width 0.2) (layer "F.Cu") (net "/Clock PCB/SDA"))
 (segment (start 121.325 89.2) (end 121.325 76.25) (width 0.2) (layer "F.Cu") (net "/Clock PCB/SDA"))
 (segment (start 120.975 89.55) (end 121.325 89.2) (width 0.2) (layer "F.Cu") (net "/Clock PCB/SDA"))
 (segment (start 109.465 101.205627) (end 111.394373 101.205627) (width 0.2) (layer "F.Cu") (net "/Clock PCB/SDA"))
 (segment (start 135.195 64.055) (end 134.65 63.51) (width 0.2) (layer "F.Cu") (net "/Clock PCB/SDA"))
 (segment (start 129.57 72.8) (end 135.195 67.175) (width 0.2) (layer "F.Cu") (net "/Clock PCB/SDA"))
 (segment (start 124.775 72.8) (end 129.57 72.8) (width 0.2) (layer "F.Cu") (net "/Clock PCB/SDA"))
 (segment (start 109.465 113.205627) (end 112.525 113.205627) (width 0.2) (layer "F.Cu") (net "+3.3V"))
 (segment (start 132.825 62.49) (end 132.8 62.465) (width 0.2) (layer "F.Cu") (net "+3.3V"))
 (segment (start 130.115 65.15) (end 130.115 67.175) (width 0.2) (layer "F.Cu") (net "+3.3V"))
 (segment (start 130.115 63.69) (end 130.115 65.15) (width 0.2) (layer "F.Cu") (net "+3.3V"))
 (segment (start 132.8 62.465) (end 130.115 65.15) (width 0.2) (layer "F.Cu") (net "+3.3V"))
 (segment (start 123.1 51.01) (end 123.1 53.1) (width 0.2) (layer "F.Cu") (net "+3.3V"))
 (segment (start 129.4 62.975) (end 130.115 63.69) (width 0.2) (layer "F.Cu") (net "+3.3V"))
 (segment (start 123.1 53.1) (end 131.2825 61.2825) (width 0.2) (layer "F.Cu") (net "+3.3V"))
 (segment (start 129.4 61.525) (end 129.4 62.975) (width 0.2) (layer "F.Cu") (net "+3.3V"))
 (segment (start 132 154.465) (end 132 130.680627) (width 0.2) (layer "F.Cu") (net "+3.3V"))
 (segment (start 132 130.680627) (end 113.525 112.205627) (width 0.2) (layer "F.Cu") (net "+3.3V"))
 (segment (start 129.025 61.15) (end 129.4 61.525) (width 0.2) (layer "F.Cu") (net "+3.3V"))
 (segment (start 131.2825 61.2825) (end 131.2825 63.9825) (width 0.2) (layer "F.Cu") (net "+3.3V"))
 (segment (start 129.4 62.975) (end 129.375 62.975) (width 0.2) (layer "F.Cu") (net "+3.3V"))
 (segment (start 134.65 62.49) (end 132.825 62.49) (width 0.2) (layer "F.Cu") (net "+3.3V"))
 (segment (start 112.525 113.205627) (end 113.525 112.205627) (width 0.2) (layer "F.Cu") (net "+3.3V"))
 (via (at 113.525 112.205627) (size 0.6) (drill 0.3) (layers "F.Cu" "B.Cu") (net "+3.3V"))
 (segment (start 129.95 93.275) (end 129.95 67.34) (width 0.2) (layer "B.Cu") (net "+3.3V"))
 (segment (start 114.95 110.780627) (end 114.95 108.275) (width 0.2) (layer "B.Cu") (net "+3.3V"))
 (segment (start 129.95 67.34) (end 130.115 67.175) (width 0.2) (layer "B.Cu") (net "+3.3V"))
 (segment (start 113.525 112.205627) (end 114.95 110.780627) (width 0.2) (layer "B.Cu") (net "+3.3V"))
 (segment (start 114.95 108.275) (end 129.95 93.275) (width 0.2) (layer "B.Cu") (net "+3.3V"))
 (segment (start 115.225 97.325) (end 115.25 97.3) (width 0.2) (layer "F.Cu") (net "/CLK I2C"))
 (segment (start 123.675 69.775) (end 115.25 78.2) (width 0.2) (layer "F.Cu") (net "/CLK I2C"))
 (segment (start 130.055 69.775) (end 123.675 69.775) (width 0.2) (layer "F.Cu") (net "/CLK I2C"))
 (segment (start 115.225 99.65) (end 115.225 97.325) (width 0.2) (layer "F.Cu") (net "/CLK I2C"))
 (segment (start 132.8 67.03) (end 132.655 67.175) (width 0.2) (layer "F.Cu") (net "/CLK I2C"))
 (segment (start 115.25 78.2) (end 115.25 93.45) (width 0.2) (layer "F.Cu") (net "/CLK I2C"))
 (segment (start 132.655 67.175) (end 130.055 69.775) (width 0.2) (layer "F.Cu") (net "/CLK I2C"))
 (segment (start 109.534373 102.275) (end 112.6 102.275) (width 0.2) (layer "F.Cu") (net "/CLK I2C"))
 (segment (start 109.465 102.205627) (end 109.534373 102.275) (width 0.2) (layer "F.Cu") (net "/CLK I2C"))
 (segment (start 112.6 102.275) (end 115.225 99.65) (width 0.2) (layer "F.Cu") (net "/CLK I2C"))
 (segment (start 132.8 63.485) (end 132.8 67.03) (width 0.2) (layer "F.Cu") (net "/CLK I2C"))
 (via (at 115.25 93.45) (size 0.6) (drill 0.3) (layers "F.Cu" "B.Cu") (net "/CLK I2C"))
 (via (at 115.25 97.3) (size 0.6) (drill 0.3) (layers "F.Cu" "B.Cu") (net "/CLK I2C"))
 (segment (start 115.25 97.3) (end 115.25 93.45) (width 0.2) (layer "B.Cu") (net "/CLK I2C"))
 (segment (start 123.1 49.99) (end 123.515627 49.99) (width 0.2) (layer "F.Cu") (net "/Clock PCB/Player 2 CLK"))
 (segment (start 111.125 100.205627) (end 112.225 99.105627) (width 0.2) (layer "F.Cu") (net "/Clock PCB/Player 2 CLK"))
 (segment (start 120.575 48.755627) (end 124.75 48.755627) (width 0.2) (layer "F.Cu") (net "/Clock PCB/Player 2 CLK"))
 (segment (start 112.225 57.105627) (end 120.575 48.755627) (width 0.2) (layer "F.Cu") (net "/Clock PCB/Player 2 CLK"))
 (segment (start 124.75 48.755627) (end 126.895 48.755627) (width 0.2) (layer "F.Cu") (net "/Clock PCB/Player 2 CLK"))
 (segment (start 109.465 100.205627) (end 111.125 100.205627) (width 0.2) (layer "F.Cu") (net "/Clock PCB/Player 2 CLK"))
 (segment (start 123.515627 49.99) (end 124.75 48.755627) (width 0.2) (layer "F.Cu") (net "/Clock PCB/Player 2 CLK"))
 (segment (start 112.225 99.105627) (end 112.225 57.105627) (width 0.2) (layer "F.Cu") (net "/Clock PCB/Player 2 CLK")))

